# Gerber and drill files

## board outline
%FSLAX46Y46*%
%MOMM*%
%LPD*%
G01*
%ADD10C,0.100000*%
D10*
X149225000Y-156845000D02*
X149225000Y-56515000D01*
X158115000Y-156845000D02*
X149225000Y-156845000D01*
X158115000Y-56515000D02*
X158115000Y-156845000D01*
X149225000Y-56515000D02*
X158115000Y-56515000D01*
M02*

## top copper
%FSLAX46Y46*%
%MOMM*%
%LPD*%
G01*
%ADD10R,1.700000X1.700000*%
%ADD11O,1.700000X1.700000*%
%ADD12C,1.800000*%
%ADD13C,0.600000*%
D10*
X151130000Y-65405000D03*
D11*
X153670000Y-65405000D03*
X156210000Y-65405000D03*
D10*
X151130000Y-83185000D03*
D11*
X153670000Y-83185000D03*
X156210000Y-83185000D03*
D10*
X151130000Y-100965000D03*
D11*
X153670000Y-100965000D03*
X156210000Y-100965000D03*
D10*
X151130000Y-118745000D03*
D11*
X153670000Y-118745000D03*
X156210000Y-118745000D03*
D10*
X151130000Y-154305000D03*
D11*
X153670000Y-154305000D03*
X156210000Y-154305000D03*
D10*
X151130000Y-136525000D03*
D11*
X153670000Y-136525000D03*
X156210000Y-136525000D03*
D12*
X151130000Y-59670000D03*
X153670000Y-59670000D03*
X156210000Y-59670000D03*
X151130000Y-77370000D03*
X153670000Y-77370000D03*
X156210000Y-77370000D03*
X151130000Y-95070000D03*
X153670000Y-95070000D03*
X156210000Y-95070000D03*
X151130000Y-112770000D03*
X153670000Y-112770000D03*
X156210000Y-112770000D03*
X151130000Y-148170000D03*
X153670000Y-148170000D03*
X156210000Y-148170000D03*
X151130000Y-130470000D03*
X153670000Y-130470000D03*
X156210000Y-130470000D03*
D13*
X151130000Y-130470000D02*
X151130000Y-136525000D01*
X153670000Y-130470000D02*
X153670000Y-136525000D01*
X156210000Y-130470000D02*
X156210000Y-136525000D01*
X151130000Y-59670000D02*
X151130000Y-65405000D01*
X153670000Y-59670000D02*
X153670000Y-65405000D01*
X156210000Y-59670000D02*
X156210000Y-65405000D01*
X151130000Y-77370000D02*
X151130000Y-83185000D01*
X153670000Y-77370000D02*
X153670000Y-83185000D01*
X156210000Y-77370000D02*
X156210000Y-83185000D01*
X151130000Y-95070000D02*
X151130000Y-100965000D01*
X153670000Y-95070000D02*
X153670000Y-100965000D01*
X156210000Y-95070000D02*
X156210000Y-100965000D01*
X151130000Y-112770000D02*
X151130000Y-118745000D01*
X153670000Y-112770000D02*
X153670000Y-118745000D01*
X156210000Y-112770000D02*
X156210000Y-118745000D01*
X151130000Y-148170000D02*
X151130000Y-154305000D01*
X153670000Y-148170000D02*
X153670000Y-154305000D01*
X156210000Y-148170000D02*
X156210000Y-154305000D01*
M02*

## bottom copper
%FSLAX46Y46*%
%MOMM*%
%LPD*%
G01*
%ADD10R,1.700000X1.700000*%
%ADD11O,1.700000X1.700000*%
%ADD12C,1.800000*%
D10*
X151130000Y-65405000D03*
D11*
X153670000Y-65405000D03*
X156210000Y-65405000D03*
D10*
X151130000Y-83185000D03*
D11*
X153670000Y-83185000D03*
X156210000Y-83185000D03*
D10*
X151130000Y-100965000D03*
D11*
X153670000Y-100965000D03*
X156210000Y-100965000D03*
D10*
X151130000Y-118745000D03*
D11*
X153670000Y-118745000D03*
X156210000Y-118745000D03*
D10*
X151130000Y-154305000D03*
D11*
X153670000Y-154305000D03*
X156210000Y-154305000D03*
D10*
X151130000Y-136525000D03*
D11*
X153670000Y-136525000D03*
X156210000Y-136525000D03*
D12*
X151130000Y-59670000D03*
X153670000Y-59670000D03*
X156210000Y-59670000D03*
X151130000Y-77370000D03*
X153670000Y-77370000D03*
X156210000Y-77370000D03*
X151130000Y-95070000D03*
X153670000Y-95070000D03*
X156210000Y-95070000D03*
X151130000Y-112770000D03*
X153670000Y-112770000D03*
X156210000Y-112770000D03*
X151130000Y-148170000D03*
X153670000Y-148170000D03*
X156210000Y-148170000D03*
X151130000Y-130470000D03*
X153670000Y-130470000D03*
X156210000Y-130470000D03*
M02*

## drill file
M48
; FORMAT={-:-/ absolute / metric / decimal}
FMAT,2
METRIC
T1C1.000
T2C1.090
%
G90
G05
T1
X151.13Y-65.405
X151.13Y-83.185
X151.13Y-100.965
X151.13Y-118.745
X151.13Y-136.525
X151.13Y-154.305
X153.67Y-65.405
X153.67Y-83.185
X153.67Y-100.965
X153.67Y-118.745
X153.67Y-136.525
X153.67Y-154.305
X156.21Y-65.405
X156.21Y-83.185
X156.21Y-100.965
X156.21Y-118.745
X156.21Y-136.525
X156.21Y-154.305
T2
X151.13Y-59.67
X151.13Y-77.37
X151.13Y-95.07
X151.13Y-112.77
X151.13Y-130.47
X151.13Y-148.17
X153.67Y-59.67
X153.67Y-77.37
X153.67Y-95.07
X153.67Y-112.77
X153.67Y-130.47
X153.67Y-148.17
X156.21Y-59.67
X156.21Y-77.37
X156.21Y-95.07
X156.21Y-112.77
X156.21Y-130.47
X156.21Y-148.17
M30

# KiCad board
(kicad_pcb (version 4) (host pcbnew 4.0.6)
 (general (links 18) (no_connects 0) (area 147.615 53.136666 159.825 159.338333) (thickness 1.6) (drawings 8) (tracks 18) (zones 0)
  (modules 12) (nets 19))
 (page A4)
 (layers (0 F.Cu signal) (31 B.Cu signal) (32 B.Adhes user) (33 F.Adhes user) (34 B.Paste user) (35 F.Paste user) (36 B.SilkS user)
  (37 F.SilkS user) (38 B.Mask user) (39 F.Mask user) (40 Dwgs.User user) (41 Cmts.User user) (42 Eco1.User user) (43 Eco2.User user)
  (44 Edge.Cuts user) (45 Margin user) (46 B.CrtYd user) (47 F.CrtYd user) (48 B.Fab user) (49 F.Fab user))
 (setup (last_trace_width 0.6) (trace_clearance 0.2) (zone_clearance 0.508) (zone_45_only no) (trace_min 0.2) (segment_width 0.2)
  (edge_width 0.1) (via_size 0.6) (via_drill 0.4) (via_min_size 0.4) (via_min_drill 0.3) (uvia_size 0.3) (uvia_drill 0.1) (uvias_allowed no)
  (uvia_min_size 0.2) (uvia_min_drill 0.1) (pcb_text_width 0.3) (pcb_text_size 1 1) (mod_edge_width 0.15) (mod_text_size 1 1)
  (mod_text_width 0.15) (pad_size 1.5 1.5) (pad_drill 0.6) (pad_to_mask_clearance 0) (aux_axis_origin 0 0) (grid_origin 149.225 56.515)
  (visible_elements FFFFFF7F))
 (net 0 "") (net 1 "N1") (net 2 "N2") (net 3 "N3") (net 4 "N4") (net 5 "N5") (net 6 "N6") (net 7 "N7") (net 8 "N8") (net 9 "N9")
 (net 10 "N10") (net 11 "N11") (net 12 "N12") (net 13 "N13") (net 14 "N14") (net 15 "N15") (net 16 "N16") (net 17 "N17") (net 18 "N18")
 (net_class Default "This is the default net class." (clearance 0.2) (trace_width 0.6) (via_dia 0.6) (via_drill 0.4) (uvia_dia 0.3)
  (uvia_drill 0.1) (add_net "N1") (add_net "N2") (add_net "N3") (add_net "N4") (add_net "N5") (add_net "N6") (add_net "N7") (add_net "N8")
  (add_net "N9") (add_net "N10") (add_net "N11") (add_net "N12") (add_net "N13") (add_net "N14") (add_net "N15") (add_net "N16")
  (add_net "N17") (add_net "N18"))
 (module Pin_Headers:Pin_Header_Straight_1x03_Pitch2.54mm (layer B.Cu) (at 151.13 65.405 270)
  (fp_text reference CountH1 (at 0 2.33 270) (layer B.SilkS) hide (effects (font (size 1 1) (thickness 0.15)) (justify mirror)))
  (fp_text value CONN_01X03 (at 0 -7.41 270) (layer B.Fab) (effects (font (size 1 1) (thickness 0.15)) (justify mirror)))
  (pad 1 thru_hole rect (at 0 0 270) (size 1.7 1.7) (drill 1) (layers *.Cu *.Mask) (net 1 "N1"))
  (pad 2 thru_hole oval (at 0 -2.54 270) (size 1.7 1.7) (drill 1) (layers *.Cu *.Mask) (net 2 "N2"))
  (pad 3 thru_hole oval (at 0 -5.08 270) (size 1.7 1.7) (drill 1) (layers *.Cu *.Mask) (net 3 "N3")))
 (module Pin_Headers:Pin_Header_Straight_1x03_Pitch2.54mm (layer B.Cu) (at 151.13 83.185 270)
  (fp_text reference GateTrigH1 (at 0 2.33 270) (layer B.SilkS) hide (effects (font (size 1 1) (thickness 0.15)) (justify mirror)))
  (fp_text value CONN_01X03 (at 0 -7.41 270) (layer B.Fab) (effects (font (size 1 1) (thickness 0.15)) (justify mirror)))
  (pad 1 thru_hole rect (at 0 0 270) (size 1.7 1.7) (drill 1) (layers *.Cu *.Mask) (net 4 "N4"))
  (pad 2 thru_hole oval (at 0 -2.54 270) (size 1.7 1.7) (drill 1) (layers *.Cu *.Mask) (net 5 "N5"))
  (pad 3 thru_hole oval (at 0 -5.08 270) (size 1.7 1.7) (drill 1) (layers *.Cu *.Mask) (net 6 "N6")))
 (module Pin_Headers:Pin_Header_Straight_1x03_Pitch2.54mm (layer B.Cu) (at 151.13 100.965 270)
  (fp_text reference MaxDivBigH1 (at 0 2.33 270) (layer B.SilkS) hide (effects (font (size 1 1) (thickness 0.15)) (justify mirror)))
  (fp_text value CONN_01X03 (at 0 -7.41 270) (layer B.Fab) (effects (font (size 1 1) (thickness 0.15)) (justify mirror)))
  (pad 1 thru_hole rect (at 0 0 270) (size 1.7 1.7) (drill 1) (layers *.Cu *.Mask) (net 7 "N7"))
  (pad 2 thru_hole oval (at 0 -2.54 270) (size 1.7 1.7) (drill 1) (layers *.Cu *.Mask) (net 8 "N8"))
  (pad 3 thru_hole oval (at 0 -5.08 270) (size 1.7 1.7) (drill 1) (layers *.Cu *.Mask) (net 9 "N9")))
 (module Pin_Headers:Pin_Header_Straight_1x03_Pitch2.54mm (layer B.Cu) (at 151.13 118.745 270)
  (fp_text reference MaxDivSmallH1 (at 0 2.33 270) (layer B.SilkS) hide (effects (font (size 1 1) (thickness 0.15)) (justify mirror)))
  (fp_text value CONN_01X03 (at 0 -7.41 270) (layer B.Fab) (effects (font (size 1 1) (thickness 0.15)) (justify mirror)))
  (pad 1 thru_hole rect (at 0 0 270) (size 1.7 1.7) (drill 1) (layers *.Cu *.Mask) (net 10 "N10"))
  (pad 2 thru_hole oval (at 0 -2.54 270) (size 1.7 1.7) (drill 1) (layers *.Cu *.Mask) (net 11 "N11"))
  (pad 3 thru_hole oval (at 0 -5.08 270) (size 1.7 1.7) (drill 1) (layers *.Cu *.Mask) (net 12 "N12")))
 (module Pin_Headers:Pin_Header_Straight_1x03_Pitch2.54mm (layer B.Cu) (at 151.13 154.305 270)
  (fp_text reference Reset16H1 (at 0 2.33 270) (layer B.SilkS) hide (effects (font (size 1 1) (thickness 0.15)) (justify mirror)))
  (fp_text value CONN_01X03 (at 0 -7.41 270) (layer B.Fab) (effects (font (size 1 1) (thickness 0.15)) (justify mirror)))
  (pad 1 thru_hole rect (at 0 0 270) (size 1.7 1.7) (drill 1) (layers *.Cu *.Mask) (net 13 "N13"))
  (pad 2 thru_hole oval (at 0 -2.54 270) (size 1.7 1.7) (drill 1) (layers *.Cu *.Mask) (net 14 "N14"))
  (pad 3 thru_hole oval (at 0 -5.08 270) (size 1.7 1.7) (drill 1) (layers *.Cu *.Mask) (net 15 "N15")))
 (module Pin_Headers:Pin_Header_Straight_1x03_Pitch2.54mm (layer B.Cu) (at 151.13 136.525 270)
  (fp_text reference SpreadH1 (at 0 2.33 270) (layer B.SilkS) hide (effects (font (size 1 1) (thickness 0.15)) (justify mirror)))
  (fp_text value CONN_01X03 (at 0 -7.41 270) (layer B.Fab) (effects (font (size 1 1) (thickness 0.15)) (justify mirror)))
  (pad 1 thru_hole rect (at 0 0 270) (size 1.7 1.7) (drill 1) (layers *.Cu *.Mask) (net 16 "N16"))
  (pad 2 thru_hole oval (at 0 -2.54 270) (size 1.7 1.7) (drill 1) (layers *.Cu *.Mask) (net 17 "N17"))
  (pad 3 thru_hole oval (at 0 -5.08 270) (size 1.7 1.7) (drill 1) (layers *.Cu *.Mask) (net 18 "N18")))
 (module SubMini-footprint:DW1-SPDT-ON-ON (layer F.Cu) (at 156.21 59.67 90)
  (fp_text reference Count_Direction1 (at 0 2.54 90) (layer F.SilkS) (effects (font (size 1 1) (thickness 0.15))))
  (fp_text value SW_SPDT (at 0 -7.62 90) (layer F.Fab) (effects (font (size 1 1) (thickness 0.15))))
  (pad 1 thru_hole circle (at 0 -5.08 90) (size 1.8 1.8) (drill 1.09) (layers *.Cu *.Mask) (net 1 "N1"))
  (pad 2 thru_hole circle (at 0 -2.54 90) (size 1.8 1.8) (drill 1.09) (layers *.Cu *.Mask) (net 2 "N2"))
  (pad 3 thru_hole circle (at 0 0 90) (size 1.8 1.8) (drill 1.09) (layers *.Cu *.Mask) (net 3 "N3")))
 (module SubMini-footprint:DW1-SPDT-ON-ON (layer F.Cu) (at 156.21 77.37 90)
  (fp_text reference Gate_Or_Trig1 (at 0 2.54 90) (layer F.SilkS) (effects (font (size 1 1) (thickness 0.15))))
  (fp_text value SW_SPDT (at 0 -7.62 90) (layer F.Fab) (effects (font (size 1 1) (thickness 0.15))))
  (pad 1 thru_hole circle (at 0 -5.08 90) (size 1.8 1.8) (drill 1.09) (layers *.Cu *.Mask) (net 4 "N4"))
  (pad 2 thru_hole circle (at 0 -2.54 90) (size 1.8 1.8) (drill 1.09) (layers *.Cu *.Mask) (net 5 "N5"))
  (pad 3 thru_hole circle (at 0 0 90) (size 1.8 1.8) (drill 1.09) (layers *.Cu *.Mask) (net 6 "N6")))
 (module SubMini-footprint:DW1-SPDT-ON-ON (layer F.Cu) (at 156.21 95.07 90)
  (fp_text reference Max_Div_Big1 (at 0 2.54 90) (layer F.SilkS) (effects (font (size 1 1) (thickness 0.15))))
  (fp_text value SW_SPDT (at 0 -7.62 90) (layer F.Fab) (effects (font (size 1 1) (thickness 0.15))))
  (pad 1 thru_hole circle (at 0 -5.08 90) (size 1.8 1.8) (drill 1.09) (layers *.Cu *.Mask) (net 7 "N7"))
  (pad 2 thru_hole circle (at 0 -2.54 90) (size 1.8 1.8) (drill 1.09) (layers *.Cu *.Mask) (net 8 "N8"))
  (pad 3 thru_hole circle (at 0 0 90) (size 1.8 1.8) (drill 1.09) (layers *.Cu *.Mask) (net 9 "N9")))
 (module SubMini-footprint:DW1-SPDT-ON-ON (layer F.Cu) (at 156.21 112.77 90)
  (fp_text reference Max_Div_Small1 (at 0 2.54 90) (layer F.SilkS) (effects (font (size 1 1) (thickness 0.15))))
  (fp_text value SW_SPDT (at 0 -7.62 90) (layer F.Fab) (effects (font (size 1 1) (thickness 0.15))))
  (pad 1 thru_hole circle (at 0 -5.08 90) (size 1.8 1.8) (drill 1.09) (layers *.Cu *.Mask) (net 10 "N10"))
  (pad 2 thru_hole circle (at 0 -2.54 90) (size 1.8 1.8) (drill 1.09) (layers *.Cu *.Mask) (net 11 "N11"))
  (pad 3 thru_hole circle (at 0 0 90) (size 1.8 1.8) (drill 1.09) (layers *.Cu *.Mask) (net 12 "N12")))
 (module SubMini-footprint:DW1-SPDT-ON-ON (layer F.Cu) (at 156.21 148.17 90)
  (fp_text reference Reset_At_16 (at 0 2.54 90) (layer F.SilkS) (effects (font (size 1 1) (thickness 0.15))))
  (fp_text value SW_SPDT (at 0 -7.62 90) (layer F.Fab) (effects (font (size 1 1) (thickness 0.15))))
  (pad 1 thru_hole circle (at 0 -5.08 90) (size 1.8 1.8) (drill 1.09) (layers *.Cu *.Mask) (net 13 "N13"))
  (pad 2 thru_hole circle (at 0 -2.54 90) (size 1.8 1.8) (drill 1.09) (layers *.Cu *.Mask) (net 14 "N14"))
  (pad 3 thru_hole circle (at 0 0 90) (size 1.8 1.8) (drill 1.09) (layers *.Cu *.Mask) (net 15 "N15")))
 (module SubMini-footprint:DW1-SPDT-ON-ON (layer F.Cu) (at 156.21 130.47 90)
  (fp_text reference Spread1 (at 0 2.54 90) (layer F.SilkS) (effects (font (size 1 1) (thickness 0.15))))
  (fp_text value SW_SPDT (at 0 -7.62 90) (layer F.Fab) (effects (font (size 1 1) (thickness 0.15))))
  (pad 1 thru_hole circle (at 0 -5.08 90) (size 1.8 1.8) (drill 1.09) (layers *.Cu *.Mask) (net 16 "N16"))
  (pad 2 thru_hole circle (at 0 -2.54 90) (size 1.8 1.8) (drill 1.09) (layers *.Cu *.Mask) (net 17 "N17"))
  (pad 3 thru_hole circle (at 0 0 90) (size 1.8 1.8) (drill 1.09) (layers *.Cu *.Mask) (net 18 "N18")))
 (gr_line (start 149.225 156.845) (end 149.225 56.515) (angle 90) (layer Edge.Cuts) (width 0.1))
 (gr_line (start 158.115 156.845) (end 149.225 156.845) (angle 90) (layer Edge.Cuts) (width 0.1))
 (gr_line (start 158.115 56.515) (end 158.115 156.845) (angle 90) (layer Edge.Cuts) (width 0.1))
 (gr_line (start 149.225 56.515) (end 158.115 56.515) (angle 90) (layer Edge.Cuts) (width 0.1))
 (segment (start 151.13 130.47) (end 151.13 136.525) (width 0.6) (layer F.Cu) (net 16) (status 20))
 (segment (start 153.67 130.47) (end 153.67 136.525) (width 0.6) (layer F.Cu) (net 17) (status 20))
 (segment (start 156.21 130.47) (end 156.21 136.525) (width 0.6) (layer F.Cu) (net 18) (status 20))
 (segment (start 151.13 59.67) (end 151.13 65.405) (width 0.6) (layer F.Cu) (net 1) (status 20))
 (segment (start 153.67 59.67) (end 153.67 65.405) (width 0.6) (layer F.Cu) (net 2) (status 20))
 (segment (start 156.21 59.67) (end 156.21 65.405) (width 0.6) (layer F.Cu) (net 3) (status 20))
 (segment (start 151.13 77.37) (end 151.13 83.185) (width 0.6) (layer F.Cu) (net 4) (status 20))
 (segment (start 153.67 77.37) (end 153.67 83.185) (width 0.6) (layer F.Cu) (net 5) (status 20))
 (segment (start 156.21 77.37) (end 156.21 83.185) (width 0.6) (layer F.Cu) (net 6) (status 20))
 (segment (start 151.13 95.07) (end 151.13 100.965) (width 0.6) (layer F.Cu) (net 7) (status 20))
 (segment (start 153.67 95.07) (end 153.67 100.965) (width 0.6) (layer F.Cu) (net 8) (status 20))
 (segment (start 156.21 95.07) (end 156.21 100.965) (width 0.6) (layer F.Cu) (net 9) (status 20))
 (segment (start 151.13 112.77) (end 151.13 118.745) (width 0.6) (layer F.Cu) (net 10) (status 20))
 (segment (start 153.67 112.77) (end 153.67 118.745) (width 0.6) (layer F.Cu) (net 11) (status 20))
 (segment (start 156.21 112.77) (end 156.21 118.745) (width 0.6) (layer F.Cu) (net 12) (status 20))
 (segment (start 151.13 148.17) (end 151.13 154.305) (width 0.6) (layer F.Cu) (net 13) (status 20))
 (segment (start 153.67 148.17) (end 153.67 154.305) (width 0.6) (layer F.Cu) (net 14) (status 20))
 (segment (start 156.21 148.17) (end 156.21 154.305) (width 0.6) (layer F.Cu) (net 15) (status 20)))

